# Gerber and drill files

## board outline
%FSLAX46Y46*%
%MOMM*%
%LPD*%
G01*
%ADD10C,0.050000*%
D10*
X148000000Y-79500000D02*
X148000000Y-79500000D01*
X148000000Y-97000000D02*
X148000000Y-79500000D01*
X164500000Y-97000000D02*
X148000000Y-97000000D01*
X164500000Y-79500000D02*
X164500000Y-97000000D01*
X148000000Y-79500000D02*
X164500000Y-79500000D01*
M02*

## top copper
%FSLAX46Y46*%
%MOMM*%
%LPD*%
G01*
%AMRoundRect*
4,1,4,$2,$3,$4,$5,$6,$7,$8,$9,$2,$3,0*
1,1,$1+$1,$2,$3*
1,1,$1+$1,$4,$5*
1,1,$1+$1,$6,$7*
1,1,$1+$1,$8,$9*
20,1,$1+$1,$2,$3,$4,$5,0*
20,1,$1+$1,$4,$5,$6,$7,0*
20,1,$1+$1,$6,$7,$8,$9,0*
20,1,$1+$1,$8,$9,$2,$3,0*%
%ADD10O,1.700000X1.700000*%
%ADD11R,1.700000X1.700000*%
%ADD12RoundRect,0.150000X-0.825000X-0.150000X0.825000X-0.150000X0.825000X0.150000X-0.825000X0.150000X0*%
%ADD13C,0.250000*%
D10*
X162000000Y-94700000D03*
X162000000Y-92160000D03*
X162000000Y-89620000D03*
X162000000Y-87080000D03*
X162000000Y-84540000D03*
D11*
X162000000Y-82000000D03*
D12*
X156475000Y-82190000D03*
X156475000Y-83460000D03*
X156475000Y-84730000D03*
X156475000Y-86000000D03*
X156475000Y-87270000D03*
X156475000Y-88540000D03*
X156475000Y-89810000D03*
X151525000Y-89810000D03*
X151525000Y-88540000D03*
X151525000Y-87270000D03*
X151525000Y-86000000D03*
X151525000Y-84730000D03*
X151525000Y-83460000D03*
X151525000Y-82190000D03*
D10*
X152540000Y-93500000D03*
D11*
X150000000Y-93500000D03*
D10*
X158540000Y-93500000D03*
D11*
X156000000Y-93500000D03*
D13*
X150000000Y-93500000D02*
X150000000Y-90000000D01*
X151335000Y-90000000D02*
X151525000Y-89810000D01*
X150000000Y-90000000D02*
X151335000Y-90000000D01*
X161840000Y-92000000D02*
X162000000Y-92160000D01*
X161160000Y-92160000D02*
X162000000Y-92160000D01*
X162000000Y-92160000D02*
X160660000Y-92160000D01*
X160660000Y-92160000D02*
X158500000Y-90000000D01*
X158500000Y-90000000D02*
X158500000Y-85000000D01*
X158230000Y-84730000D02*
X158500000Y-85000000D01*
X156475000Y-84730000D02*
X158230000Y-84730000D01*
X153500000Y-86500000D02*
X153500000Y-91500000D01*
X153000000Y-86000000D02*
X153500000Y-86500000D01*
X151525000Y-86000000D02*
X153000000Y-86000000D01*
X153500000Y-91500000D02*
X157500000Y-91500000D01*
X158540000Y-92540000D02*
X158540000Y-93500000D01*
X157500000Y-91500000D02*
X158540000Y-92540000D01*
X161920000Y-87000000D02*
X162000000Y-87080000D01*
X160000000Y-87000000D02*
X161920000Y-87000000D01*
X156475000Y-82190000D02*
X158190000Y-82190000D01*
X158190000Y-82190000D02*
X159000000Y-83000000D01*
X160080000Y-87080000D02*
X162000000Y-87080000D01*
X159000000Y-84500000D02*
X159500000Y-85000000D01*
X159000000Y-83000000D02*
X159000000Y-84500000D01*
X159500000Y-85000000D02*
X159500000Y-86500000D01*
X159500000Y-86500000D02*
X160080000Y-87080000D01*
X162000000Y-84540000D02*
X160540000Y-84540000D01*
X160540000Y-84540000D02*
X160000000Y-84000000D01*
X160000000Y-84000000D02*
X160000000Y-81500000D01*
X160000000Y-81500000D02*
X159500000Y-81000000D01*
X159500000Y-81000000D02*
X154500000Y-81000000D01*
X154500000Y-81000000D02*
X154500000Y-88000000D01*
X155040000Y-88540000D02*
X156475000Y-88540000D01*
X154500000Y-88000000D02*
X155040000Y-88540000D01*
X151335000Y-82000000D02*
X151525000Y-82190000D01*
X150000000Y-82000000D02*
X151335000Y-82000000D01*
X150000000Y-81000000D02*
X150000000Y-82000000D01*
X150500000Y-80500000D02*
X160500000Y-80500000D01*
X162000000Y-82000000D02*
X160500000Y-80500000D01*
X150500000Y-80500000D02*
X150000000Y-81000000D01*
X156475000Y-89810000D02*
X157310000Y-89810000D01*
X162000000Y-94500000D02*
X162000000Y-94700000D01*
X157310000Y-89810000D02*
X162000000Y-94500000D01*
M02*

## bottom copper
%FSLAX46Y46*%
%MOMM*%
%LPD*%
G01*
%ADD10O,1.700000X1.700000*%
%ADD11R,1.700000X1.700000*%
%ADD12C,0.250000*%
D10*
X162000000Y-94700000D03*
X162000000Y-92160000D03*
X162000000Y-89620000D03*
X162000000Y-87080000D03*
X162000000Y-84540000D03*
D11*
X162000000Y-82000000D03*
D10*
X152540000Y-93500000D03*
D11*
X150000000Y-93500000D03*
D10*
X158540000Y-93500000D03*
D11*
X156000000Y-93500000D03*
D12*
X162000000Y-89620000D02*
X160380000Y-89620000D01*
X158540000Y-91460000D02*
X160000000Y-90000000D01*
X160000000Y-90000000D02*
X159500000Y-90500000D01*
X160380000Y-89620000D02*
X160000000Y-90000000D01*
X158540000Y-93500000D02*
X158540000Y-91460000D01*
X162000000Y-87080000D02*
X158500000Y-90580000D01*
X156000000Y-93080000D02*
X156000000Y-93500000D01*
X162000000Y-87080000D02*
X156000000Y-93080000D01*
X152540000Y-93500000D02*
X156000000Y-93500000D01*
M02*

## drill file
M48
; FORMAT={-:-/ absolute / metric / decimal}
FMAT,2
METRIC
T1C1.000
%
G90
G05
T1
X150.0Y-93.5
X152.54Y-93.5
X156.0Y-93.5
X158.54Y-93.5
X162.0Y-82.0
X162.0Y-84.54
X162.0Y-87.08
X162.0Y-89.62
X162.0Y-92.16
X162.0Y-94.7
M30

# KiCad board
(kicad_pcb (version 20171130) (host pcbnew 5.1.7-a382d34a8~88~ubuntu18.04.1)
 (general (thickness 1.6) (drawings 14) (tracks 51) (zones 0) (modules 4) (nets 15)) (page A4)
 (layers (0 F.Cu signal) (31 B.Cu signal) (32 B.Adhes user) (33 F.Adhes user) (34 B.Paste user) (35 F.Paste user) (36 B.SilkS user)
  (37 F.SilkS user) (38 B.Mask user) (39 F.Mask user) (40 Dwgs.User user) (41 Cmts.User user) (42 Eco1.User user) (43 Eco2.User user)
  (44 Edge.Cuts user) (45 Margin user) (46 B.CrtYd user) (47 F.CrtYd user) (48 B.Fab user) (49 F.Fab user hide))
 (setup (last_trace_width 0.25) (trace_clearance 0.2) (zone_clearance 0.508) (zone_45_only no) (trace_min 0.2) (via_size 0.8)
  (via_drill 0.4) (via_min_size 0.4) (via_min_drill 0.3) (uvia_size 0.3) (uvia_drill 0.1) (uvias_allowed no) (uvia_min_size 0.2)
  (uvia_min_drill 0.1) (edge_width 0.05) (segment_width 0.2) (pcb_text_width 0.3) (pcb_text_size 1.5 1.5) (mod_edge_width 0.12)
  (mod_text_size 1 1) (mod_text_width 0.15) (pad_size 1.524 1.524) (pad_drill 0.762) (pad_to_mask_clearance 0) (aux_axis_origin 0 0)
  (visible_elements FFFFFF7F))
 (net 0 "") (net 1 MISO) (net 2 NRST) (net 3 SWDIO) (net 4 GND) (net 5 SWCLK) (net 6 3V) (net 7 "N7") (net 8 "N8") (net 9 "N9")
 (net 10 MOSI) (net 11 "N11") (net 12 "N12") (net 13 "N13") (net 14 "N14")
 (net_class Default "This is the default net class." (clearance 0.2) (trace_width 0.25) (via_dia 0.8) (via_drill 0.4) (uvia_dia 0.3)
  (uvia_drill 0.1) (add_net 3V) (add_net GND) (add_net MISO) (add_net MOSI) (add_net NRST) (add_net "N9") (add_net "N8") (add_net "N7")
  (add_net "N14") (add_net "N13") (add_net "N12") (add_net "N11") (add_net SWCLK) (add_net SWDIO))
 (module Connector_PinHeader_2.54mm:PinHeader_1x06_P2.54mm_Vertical (layer F.Cu) (at 162 82)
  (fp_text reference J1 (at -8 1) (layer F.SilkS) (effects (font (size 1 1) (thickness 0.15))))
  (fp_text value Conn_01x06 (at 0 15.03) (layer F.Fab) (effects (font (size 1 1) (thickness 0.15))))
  (pad 6 thru_hole oval (at 0 12.7) (size 1.7 1.7) (drill 1) (layers *.Cu *.Mask) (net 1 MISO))
  (pad 5 thru_hole oval (at 0 10.16) (size 1.7 1.7) (drill 1) (layers *.Cu *.Mask) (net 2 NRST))
  (pad 4 thru_hole oval (at 0 7.62) (size 1.7 1.7) (drill 1) (layers *.Cu *.Mask) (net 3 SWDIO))
  (pad 3 thru_hole oval (at 0 5.08) (size 1.7 1.7) (drill 1) (layers *.Cu *.Mask) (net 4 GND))
  (pad 2 thru_hole oval (at 0 2.54) (size 1.7 1.7) (drill 1) (layers *.Cu *.Mask) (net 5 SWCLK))
  (pad 1 thru_hole rect (at 0 0) (size 1.7 1.7) (drill 1) (layers *.Cu *.Mask) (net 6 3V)))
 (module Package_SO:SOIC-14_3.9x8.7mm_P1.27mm (layer F.Cu) (at 154 86)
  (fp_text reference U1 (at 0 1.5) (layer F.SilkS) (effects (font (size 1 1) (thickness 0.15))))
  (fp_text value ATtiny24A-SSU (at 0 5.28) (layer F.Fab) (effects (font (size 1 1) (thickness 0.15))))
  (pad 14 smd roundrect (at 2.475 -3.81) (size 1.95 0.6) (layers F.Cu F.Paste F.Mask) (roundrect_rratio 0.25) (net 4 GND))
  (pad 13 smd roundrect (at 2.475 -2.54) (size 1.95 0.6) (layers F.Cu F.Paste F.Mask) (roundrect_rratio 0.25) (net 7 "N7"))
  (pad 12 smd roundrect (at 2.475 -1.27) (size 1.95 0.6) (layers F.Cu F.Paste F.Mask) (roundrect_rratio 0.25) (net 2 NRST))
  (pad 11 smd roundrect (at 2.475 0) (size 1.95 0.6) (layers F.Cu F.Paste F.Mask) (roundrect_rratio 0.25) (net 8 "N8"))
  (pad 10 smd roundrect (at 2.475 1.27) (size 1.95 0.6) (layers F.Cu F.Paste F.Mask) (roundrect_rratio 0.25) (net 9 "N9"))
  (pad 9 smd roundrect (at 2.475 2.54) (size 1.95 0.6) (layers F.Cu F.Paste F.Mask) (roundrect_rratio 0.25) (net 5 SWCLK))
  (pad 8 smd roundrect (at 2.475 3.81) (size 1.95 0.6) (layers F.Cu F.Paste F.Mask) (roundrect_rratio 0.25) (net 1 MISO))
  (pad 7 smd roundrect (at -2.475 3.81) (size 1.95 0.6) (layers F.Cu F.Paste F.Mask) (roundrect_rratio 0.25) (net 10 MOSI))
  (pad 6 smd roundrect (at -2.475 2.54) (size 1.95 0.6) (layers F.Cu F.Paste F.Mask) (roundrect_rratio 0.25) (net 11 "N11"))
  (pad 5 smd roundrect (at -2.475 1.27) (size 1.95 0.6) (layers F.Cu F.Paste F.Mask) (roundrect_rratio 0.25) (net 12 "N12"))
  (pad 4 smd roundrect (at -2.475 0) (size 1.95 0.6) (layers F.Cu F.Paste F.Mask) (roundrect_rratio 0.25) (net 3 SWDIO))
  (pad 3 smd roundrect (at -2.475 -1.27) (size 1.95 0.6) (layers F.Cu F.Paste F.Mask) (roundrect_rratio 0.25) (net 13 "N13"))
  (pad 2 smd roundrect (at -2.475 -2.54) (size 1.95 0.6) (layers F.Cu F.Paste F.Mask) (roundrect_rratio 0.25) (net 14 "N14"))
  (pad 1 smd roundrect (at -2.475 -3.81) (size 1.95 0.6) (layers F.Cu F.Paste F.Mask) (roundrect_rratio 0.25) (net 6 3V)))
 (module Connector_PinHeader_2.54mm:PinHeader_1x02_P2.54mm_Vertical (layer F.Cu) (at 150 93.5 90)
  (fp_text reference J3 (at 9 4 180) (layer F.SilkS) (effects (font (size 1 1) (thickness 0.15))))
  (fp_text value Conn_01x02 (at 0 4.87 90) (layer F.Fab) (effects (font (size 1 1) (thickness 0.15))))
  (pad 2 thru_hole oval (at 0 2.54 90) (size 1.7 1.7) (drill 1) (layers *.Cu *.Mask) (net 4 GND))
  (pad 1 thru_hole rect (at 0 0 90) (size 1.7 1.7) (drill 1) (layers *.Cu *.Mask) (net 10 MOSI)))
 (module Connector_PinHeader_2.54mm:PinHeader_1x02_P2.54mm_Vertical (layer F.Cu) (at 156 93.5 90)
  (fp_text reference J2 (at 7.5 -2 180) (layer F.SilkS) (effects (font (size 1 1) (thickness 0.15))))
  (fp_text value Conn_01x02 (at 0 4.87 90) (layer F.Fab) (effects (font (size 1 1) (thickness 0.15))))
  (pad 2 thru_hole oval (at 0 2.54 90) (size 1.7 1.7) (drill 1) (layers *.Cu *.Mask) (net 3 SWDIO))
  (pad 1 thru_hole rect (at 0 0 90) (size 1.7 1.7) (drill 1) (layers *.Cu *.Mask) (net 4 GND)))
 (gr_line (start 148 79.5) (end 148 79.5) (layer Edge.Cuts) (width 0.05))
 (gr_line (start 148 97) (end 148 79.5) (layer Edge.Cuts) (width 0.05))
 (gr_line (start 164.5 97) (end 148 97) (layer Edge.Cuts) (width 0.05))
 (gr_line (start 164.5 79.5) (end 164.5 97) (layer Edge.Cuts) (width 0.05))
 (gr_line (start 148 79.5) (end 164.5 79.5) (layer Edge.Cuts) (width 0.05))
 (segment (start 150 93.5) (end 150 90) (width 0.25) (layer F.Cu) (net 10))
 (segment (start 151.335 90) (end 151.525 89.81) (width 0.25) (layer F.Cu) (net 10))
 (segment (start 150 90) (end 151.335 90) (width 0.25) (layer F.Cu) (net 10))
 (segment (start 161.84 92) (end 162 92.16) (width 0.25) (layer F.Cu) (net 2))
 (segment (start 161.16 92.16) (end 162 92.16) (width 0.25) (layer F.Cu) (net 2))
 (segment (start 162 92.16) (end 160.66 92.16) (width 0.25) (layer F.Cu) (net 2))
 (segment (start 160.66 92.16) (end 158.5 90) (width 0.25) (layer F.Cu) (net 2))
 (segment (start 158.5 90) (end 158.5 85) (width 0.25) (layer F.Cu) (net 2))
 (segment (start 158.23 84.73) (end 158.5 85) (width 0.25) (layer F.Cu) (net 2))
 (segment (start 156.475 84.73) (end 158.23 84.73) (width 0.25) (layer F.Cu) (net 2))
 (segment (start 162 89.62) (end 160.38 89.62) (width 0.25) (layer B.Cu) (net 3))
 (segment (start 158.54 91.46) (end 160 90) (width 0.25) (layer B.Cu) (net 3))
 (segment (start 160 90) (end 159.5 90.5) (width 0.25) (layer B.Cu) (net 3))
 (segment (start 160.38 89.62) (end 160 90) (width 0.25) (layer B.Cu) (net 3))
 (segment (start 153.5 86.5) (end 153.5 91.5) (width 0.25) (layer F.Cu) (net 3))
 (segment (start 153 86) (end 153.5 86.5) (width 0.25) (layer F.Cu) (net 3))
 (segment (start 151.525 86) (end 153 86) (width 0.25) (layer F.Cu) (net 3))
 (segment (start 158.54 93.5) (end 158.54 91.46) (width 0.25) (layer B.Cu) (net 3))
 (segment (start 153.5 91.5) (end 157.5 91.5) (width 0.25) (layer F.Cu) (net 3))
 (segment (start 158.54 92.54) (end 158.54 93.5) (width 0.25) (layer F.Cu) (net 3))
 (segment (start 157.5 91.5) (end 158.54 92.54) (width 0.25) (layer F.Cu) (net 3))
 (segment (start 161.92 87) (end 162 87.08) (width 0.25) (layer F.Cu) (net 4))
 (segment (start 160 87) (end 161.92 87) (width 0.25) (layer F.Cu) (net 4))
 (segment (start 156.475 82.19) (end 158.19 82.19) (width 0.25) (layer F.Cu) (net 4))
 (segment (start 158.19 82.19) (end 159 83) (width 0.25) (layer F.Cu) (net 4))
 (segment (start 160.08 87.08) (end 162 87.08) (width 0.25) (layer F.Cu) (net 4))
 (segment (start 162 87.08) (end 158.5 90.58) (width 0.25) (layer B.Cu) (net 4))
 (segment (start 159 84.5) (end 159.5 85) (width 0.25) (layer F.Cu) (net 4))
 (segment (start 159 83) (end 159 84.5) (width 0.25) (layer F.Cu) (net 4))
 (segment (start 159.5 85) (end 159.5 86.5) (width 0.25) (layer F.Cu) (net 4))
 (segment (start 159.5 86.5) (end 160.08 87.08) (width 0.25) (layer F.Cu) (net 4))
 (segment (start 156 93.08) (end 156 93.5) (width 0.25) (layer B.Cu) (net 4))
 (segment (start 162 87.08) (end 156 93.08) (width 0.25) (layer B.Cu) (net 4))
 (segment (start 152.54 93.5) (end 156 93.5) (width 0.25) (layer B.Cu) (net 4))
 (segment (start 162 84.54) (end 160.54 84.54) (width 0.25) (layer F.Cu) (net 5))
 (segment (start 160.54 84.54) (end 160 84) (width 0.25) (layer F.Cu) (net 5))
 (segment (start 160 84) (end 160 81.5) (width 0.25) (layer F.Cu) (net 5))
 (segment (start 160 81.5) (end 159.5 81) (width 0.25) (layer F.Cu) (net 5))
 (segment (start 159.5 81) (end 154.5 81) (width 0.25) (layer F.Cu) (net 5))
 (segment (start 154.5 81) (end 154.5 88) (width 0.25) (layer F.Cu) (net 5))
 (segment (start 155.04 88.54) (end 156.475 88.54) (width 0.25) (layer F.Cu) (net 5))
 (segment (start 154.5 88) (end 155.04 88.54) (width 0.25) (layer F.Cu) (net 5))
 (segment (start 151.335 82) (end 151.525 82.19) (width 0.25) (layer F.Cu) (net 6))
 (segment (start 150 82) (end 151.335 82) (width 0.25) (layer F.Cu) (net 6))
 (segment (start 150 81) (end 150 82) (width 0.25) (layer F.Cu) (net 6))
 (segment (start 150.5 80.5) (end 160.5 80.5) (width 0.25) (layer F.Cu) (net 6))
 (segment (start 162 82) (end 160.5 80.5) (width 0.25) (layer F.Cu) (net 6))
 (segment (start 150.5 80.5) (end 150 81) (width 0.25) (layer F.Cu) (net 6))
 (segment (start 156.475 89.81) (end 157.31 89.81) (width 0.25) (layer F.Cu) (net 1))
 (segment (start 162 94.5) (end 162 94.7) (width 0.25) (layer F.Cu) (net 1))
 (segment (start 157.31 89.81) (end 162 94.5) (width 0.25) (layer F.Cu) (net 1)))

